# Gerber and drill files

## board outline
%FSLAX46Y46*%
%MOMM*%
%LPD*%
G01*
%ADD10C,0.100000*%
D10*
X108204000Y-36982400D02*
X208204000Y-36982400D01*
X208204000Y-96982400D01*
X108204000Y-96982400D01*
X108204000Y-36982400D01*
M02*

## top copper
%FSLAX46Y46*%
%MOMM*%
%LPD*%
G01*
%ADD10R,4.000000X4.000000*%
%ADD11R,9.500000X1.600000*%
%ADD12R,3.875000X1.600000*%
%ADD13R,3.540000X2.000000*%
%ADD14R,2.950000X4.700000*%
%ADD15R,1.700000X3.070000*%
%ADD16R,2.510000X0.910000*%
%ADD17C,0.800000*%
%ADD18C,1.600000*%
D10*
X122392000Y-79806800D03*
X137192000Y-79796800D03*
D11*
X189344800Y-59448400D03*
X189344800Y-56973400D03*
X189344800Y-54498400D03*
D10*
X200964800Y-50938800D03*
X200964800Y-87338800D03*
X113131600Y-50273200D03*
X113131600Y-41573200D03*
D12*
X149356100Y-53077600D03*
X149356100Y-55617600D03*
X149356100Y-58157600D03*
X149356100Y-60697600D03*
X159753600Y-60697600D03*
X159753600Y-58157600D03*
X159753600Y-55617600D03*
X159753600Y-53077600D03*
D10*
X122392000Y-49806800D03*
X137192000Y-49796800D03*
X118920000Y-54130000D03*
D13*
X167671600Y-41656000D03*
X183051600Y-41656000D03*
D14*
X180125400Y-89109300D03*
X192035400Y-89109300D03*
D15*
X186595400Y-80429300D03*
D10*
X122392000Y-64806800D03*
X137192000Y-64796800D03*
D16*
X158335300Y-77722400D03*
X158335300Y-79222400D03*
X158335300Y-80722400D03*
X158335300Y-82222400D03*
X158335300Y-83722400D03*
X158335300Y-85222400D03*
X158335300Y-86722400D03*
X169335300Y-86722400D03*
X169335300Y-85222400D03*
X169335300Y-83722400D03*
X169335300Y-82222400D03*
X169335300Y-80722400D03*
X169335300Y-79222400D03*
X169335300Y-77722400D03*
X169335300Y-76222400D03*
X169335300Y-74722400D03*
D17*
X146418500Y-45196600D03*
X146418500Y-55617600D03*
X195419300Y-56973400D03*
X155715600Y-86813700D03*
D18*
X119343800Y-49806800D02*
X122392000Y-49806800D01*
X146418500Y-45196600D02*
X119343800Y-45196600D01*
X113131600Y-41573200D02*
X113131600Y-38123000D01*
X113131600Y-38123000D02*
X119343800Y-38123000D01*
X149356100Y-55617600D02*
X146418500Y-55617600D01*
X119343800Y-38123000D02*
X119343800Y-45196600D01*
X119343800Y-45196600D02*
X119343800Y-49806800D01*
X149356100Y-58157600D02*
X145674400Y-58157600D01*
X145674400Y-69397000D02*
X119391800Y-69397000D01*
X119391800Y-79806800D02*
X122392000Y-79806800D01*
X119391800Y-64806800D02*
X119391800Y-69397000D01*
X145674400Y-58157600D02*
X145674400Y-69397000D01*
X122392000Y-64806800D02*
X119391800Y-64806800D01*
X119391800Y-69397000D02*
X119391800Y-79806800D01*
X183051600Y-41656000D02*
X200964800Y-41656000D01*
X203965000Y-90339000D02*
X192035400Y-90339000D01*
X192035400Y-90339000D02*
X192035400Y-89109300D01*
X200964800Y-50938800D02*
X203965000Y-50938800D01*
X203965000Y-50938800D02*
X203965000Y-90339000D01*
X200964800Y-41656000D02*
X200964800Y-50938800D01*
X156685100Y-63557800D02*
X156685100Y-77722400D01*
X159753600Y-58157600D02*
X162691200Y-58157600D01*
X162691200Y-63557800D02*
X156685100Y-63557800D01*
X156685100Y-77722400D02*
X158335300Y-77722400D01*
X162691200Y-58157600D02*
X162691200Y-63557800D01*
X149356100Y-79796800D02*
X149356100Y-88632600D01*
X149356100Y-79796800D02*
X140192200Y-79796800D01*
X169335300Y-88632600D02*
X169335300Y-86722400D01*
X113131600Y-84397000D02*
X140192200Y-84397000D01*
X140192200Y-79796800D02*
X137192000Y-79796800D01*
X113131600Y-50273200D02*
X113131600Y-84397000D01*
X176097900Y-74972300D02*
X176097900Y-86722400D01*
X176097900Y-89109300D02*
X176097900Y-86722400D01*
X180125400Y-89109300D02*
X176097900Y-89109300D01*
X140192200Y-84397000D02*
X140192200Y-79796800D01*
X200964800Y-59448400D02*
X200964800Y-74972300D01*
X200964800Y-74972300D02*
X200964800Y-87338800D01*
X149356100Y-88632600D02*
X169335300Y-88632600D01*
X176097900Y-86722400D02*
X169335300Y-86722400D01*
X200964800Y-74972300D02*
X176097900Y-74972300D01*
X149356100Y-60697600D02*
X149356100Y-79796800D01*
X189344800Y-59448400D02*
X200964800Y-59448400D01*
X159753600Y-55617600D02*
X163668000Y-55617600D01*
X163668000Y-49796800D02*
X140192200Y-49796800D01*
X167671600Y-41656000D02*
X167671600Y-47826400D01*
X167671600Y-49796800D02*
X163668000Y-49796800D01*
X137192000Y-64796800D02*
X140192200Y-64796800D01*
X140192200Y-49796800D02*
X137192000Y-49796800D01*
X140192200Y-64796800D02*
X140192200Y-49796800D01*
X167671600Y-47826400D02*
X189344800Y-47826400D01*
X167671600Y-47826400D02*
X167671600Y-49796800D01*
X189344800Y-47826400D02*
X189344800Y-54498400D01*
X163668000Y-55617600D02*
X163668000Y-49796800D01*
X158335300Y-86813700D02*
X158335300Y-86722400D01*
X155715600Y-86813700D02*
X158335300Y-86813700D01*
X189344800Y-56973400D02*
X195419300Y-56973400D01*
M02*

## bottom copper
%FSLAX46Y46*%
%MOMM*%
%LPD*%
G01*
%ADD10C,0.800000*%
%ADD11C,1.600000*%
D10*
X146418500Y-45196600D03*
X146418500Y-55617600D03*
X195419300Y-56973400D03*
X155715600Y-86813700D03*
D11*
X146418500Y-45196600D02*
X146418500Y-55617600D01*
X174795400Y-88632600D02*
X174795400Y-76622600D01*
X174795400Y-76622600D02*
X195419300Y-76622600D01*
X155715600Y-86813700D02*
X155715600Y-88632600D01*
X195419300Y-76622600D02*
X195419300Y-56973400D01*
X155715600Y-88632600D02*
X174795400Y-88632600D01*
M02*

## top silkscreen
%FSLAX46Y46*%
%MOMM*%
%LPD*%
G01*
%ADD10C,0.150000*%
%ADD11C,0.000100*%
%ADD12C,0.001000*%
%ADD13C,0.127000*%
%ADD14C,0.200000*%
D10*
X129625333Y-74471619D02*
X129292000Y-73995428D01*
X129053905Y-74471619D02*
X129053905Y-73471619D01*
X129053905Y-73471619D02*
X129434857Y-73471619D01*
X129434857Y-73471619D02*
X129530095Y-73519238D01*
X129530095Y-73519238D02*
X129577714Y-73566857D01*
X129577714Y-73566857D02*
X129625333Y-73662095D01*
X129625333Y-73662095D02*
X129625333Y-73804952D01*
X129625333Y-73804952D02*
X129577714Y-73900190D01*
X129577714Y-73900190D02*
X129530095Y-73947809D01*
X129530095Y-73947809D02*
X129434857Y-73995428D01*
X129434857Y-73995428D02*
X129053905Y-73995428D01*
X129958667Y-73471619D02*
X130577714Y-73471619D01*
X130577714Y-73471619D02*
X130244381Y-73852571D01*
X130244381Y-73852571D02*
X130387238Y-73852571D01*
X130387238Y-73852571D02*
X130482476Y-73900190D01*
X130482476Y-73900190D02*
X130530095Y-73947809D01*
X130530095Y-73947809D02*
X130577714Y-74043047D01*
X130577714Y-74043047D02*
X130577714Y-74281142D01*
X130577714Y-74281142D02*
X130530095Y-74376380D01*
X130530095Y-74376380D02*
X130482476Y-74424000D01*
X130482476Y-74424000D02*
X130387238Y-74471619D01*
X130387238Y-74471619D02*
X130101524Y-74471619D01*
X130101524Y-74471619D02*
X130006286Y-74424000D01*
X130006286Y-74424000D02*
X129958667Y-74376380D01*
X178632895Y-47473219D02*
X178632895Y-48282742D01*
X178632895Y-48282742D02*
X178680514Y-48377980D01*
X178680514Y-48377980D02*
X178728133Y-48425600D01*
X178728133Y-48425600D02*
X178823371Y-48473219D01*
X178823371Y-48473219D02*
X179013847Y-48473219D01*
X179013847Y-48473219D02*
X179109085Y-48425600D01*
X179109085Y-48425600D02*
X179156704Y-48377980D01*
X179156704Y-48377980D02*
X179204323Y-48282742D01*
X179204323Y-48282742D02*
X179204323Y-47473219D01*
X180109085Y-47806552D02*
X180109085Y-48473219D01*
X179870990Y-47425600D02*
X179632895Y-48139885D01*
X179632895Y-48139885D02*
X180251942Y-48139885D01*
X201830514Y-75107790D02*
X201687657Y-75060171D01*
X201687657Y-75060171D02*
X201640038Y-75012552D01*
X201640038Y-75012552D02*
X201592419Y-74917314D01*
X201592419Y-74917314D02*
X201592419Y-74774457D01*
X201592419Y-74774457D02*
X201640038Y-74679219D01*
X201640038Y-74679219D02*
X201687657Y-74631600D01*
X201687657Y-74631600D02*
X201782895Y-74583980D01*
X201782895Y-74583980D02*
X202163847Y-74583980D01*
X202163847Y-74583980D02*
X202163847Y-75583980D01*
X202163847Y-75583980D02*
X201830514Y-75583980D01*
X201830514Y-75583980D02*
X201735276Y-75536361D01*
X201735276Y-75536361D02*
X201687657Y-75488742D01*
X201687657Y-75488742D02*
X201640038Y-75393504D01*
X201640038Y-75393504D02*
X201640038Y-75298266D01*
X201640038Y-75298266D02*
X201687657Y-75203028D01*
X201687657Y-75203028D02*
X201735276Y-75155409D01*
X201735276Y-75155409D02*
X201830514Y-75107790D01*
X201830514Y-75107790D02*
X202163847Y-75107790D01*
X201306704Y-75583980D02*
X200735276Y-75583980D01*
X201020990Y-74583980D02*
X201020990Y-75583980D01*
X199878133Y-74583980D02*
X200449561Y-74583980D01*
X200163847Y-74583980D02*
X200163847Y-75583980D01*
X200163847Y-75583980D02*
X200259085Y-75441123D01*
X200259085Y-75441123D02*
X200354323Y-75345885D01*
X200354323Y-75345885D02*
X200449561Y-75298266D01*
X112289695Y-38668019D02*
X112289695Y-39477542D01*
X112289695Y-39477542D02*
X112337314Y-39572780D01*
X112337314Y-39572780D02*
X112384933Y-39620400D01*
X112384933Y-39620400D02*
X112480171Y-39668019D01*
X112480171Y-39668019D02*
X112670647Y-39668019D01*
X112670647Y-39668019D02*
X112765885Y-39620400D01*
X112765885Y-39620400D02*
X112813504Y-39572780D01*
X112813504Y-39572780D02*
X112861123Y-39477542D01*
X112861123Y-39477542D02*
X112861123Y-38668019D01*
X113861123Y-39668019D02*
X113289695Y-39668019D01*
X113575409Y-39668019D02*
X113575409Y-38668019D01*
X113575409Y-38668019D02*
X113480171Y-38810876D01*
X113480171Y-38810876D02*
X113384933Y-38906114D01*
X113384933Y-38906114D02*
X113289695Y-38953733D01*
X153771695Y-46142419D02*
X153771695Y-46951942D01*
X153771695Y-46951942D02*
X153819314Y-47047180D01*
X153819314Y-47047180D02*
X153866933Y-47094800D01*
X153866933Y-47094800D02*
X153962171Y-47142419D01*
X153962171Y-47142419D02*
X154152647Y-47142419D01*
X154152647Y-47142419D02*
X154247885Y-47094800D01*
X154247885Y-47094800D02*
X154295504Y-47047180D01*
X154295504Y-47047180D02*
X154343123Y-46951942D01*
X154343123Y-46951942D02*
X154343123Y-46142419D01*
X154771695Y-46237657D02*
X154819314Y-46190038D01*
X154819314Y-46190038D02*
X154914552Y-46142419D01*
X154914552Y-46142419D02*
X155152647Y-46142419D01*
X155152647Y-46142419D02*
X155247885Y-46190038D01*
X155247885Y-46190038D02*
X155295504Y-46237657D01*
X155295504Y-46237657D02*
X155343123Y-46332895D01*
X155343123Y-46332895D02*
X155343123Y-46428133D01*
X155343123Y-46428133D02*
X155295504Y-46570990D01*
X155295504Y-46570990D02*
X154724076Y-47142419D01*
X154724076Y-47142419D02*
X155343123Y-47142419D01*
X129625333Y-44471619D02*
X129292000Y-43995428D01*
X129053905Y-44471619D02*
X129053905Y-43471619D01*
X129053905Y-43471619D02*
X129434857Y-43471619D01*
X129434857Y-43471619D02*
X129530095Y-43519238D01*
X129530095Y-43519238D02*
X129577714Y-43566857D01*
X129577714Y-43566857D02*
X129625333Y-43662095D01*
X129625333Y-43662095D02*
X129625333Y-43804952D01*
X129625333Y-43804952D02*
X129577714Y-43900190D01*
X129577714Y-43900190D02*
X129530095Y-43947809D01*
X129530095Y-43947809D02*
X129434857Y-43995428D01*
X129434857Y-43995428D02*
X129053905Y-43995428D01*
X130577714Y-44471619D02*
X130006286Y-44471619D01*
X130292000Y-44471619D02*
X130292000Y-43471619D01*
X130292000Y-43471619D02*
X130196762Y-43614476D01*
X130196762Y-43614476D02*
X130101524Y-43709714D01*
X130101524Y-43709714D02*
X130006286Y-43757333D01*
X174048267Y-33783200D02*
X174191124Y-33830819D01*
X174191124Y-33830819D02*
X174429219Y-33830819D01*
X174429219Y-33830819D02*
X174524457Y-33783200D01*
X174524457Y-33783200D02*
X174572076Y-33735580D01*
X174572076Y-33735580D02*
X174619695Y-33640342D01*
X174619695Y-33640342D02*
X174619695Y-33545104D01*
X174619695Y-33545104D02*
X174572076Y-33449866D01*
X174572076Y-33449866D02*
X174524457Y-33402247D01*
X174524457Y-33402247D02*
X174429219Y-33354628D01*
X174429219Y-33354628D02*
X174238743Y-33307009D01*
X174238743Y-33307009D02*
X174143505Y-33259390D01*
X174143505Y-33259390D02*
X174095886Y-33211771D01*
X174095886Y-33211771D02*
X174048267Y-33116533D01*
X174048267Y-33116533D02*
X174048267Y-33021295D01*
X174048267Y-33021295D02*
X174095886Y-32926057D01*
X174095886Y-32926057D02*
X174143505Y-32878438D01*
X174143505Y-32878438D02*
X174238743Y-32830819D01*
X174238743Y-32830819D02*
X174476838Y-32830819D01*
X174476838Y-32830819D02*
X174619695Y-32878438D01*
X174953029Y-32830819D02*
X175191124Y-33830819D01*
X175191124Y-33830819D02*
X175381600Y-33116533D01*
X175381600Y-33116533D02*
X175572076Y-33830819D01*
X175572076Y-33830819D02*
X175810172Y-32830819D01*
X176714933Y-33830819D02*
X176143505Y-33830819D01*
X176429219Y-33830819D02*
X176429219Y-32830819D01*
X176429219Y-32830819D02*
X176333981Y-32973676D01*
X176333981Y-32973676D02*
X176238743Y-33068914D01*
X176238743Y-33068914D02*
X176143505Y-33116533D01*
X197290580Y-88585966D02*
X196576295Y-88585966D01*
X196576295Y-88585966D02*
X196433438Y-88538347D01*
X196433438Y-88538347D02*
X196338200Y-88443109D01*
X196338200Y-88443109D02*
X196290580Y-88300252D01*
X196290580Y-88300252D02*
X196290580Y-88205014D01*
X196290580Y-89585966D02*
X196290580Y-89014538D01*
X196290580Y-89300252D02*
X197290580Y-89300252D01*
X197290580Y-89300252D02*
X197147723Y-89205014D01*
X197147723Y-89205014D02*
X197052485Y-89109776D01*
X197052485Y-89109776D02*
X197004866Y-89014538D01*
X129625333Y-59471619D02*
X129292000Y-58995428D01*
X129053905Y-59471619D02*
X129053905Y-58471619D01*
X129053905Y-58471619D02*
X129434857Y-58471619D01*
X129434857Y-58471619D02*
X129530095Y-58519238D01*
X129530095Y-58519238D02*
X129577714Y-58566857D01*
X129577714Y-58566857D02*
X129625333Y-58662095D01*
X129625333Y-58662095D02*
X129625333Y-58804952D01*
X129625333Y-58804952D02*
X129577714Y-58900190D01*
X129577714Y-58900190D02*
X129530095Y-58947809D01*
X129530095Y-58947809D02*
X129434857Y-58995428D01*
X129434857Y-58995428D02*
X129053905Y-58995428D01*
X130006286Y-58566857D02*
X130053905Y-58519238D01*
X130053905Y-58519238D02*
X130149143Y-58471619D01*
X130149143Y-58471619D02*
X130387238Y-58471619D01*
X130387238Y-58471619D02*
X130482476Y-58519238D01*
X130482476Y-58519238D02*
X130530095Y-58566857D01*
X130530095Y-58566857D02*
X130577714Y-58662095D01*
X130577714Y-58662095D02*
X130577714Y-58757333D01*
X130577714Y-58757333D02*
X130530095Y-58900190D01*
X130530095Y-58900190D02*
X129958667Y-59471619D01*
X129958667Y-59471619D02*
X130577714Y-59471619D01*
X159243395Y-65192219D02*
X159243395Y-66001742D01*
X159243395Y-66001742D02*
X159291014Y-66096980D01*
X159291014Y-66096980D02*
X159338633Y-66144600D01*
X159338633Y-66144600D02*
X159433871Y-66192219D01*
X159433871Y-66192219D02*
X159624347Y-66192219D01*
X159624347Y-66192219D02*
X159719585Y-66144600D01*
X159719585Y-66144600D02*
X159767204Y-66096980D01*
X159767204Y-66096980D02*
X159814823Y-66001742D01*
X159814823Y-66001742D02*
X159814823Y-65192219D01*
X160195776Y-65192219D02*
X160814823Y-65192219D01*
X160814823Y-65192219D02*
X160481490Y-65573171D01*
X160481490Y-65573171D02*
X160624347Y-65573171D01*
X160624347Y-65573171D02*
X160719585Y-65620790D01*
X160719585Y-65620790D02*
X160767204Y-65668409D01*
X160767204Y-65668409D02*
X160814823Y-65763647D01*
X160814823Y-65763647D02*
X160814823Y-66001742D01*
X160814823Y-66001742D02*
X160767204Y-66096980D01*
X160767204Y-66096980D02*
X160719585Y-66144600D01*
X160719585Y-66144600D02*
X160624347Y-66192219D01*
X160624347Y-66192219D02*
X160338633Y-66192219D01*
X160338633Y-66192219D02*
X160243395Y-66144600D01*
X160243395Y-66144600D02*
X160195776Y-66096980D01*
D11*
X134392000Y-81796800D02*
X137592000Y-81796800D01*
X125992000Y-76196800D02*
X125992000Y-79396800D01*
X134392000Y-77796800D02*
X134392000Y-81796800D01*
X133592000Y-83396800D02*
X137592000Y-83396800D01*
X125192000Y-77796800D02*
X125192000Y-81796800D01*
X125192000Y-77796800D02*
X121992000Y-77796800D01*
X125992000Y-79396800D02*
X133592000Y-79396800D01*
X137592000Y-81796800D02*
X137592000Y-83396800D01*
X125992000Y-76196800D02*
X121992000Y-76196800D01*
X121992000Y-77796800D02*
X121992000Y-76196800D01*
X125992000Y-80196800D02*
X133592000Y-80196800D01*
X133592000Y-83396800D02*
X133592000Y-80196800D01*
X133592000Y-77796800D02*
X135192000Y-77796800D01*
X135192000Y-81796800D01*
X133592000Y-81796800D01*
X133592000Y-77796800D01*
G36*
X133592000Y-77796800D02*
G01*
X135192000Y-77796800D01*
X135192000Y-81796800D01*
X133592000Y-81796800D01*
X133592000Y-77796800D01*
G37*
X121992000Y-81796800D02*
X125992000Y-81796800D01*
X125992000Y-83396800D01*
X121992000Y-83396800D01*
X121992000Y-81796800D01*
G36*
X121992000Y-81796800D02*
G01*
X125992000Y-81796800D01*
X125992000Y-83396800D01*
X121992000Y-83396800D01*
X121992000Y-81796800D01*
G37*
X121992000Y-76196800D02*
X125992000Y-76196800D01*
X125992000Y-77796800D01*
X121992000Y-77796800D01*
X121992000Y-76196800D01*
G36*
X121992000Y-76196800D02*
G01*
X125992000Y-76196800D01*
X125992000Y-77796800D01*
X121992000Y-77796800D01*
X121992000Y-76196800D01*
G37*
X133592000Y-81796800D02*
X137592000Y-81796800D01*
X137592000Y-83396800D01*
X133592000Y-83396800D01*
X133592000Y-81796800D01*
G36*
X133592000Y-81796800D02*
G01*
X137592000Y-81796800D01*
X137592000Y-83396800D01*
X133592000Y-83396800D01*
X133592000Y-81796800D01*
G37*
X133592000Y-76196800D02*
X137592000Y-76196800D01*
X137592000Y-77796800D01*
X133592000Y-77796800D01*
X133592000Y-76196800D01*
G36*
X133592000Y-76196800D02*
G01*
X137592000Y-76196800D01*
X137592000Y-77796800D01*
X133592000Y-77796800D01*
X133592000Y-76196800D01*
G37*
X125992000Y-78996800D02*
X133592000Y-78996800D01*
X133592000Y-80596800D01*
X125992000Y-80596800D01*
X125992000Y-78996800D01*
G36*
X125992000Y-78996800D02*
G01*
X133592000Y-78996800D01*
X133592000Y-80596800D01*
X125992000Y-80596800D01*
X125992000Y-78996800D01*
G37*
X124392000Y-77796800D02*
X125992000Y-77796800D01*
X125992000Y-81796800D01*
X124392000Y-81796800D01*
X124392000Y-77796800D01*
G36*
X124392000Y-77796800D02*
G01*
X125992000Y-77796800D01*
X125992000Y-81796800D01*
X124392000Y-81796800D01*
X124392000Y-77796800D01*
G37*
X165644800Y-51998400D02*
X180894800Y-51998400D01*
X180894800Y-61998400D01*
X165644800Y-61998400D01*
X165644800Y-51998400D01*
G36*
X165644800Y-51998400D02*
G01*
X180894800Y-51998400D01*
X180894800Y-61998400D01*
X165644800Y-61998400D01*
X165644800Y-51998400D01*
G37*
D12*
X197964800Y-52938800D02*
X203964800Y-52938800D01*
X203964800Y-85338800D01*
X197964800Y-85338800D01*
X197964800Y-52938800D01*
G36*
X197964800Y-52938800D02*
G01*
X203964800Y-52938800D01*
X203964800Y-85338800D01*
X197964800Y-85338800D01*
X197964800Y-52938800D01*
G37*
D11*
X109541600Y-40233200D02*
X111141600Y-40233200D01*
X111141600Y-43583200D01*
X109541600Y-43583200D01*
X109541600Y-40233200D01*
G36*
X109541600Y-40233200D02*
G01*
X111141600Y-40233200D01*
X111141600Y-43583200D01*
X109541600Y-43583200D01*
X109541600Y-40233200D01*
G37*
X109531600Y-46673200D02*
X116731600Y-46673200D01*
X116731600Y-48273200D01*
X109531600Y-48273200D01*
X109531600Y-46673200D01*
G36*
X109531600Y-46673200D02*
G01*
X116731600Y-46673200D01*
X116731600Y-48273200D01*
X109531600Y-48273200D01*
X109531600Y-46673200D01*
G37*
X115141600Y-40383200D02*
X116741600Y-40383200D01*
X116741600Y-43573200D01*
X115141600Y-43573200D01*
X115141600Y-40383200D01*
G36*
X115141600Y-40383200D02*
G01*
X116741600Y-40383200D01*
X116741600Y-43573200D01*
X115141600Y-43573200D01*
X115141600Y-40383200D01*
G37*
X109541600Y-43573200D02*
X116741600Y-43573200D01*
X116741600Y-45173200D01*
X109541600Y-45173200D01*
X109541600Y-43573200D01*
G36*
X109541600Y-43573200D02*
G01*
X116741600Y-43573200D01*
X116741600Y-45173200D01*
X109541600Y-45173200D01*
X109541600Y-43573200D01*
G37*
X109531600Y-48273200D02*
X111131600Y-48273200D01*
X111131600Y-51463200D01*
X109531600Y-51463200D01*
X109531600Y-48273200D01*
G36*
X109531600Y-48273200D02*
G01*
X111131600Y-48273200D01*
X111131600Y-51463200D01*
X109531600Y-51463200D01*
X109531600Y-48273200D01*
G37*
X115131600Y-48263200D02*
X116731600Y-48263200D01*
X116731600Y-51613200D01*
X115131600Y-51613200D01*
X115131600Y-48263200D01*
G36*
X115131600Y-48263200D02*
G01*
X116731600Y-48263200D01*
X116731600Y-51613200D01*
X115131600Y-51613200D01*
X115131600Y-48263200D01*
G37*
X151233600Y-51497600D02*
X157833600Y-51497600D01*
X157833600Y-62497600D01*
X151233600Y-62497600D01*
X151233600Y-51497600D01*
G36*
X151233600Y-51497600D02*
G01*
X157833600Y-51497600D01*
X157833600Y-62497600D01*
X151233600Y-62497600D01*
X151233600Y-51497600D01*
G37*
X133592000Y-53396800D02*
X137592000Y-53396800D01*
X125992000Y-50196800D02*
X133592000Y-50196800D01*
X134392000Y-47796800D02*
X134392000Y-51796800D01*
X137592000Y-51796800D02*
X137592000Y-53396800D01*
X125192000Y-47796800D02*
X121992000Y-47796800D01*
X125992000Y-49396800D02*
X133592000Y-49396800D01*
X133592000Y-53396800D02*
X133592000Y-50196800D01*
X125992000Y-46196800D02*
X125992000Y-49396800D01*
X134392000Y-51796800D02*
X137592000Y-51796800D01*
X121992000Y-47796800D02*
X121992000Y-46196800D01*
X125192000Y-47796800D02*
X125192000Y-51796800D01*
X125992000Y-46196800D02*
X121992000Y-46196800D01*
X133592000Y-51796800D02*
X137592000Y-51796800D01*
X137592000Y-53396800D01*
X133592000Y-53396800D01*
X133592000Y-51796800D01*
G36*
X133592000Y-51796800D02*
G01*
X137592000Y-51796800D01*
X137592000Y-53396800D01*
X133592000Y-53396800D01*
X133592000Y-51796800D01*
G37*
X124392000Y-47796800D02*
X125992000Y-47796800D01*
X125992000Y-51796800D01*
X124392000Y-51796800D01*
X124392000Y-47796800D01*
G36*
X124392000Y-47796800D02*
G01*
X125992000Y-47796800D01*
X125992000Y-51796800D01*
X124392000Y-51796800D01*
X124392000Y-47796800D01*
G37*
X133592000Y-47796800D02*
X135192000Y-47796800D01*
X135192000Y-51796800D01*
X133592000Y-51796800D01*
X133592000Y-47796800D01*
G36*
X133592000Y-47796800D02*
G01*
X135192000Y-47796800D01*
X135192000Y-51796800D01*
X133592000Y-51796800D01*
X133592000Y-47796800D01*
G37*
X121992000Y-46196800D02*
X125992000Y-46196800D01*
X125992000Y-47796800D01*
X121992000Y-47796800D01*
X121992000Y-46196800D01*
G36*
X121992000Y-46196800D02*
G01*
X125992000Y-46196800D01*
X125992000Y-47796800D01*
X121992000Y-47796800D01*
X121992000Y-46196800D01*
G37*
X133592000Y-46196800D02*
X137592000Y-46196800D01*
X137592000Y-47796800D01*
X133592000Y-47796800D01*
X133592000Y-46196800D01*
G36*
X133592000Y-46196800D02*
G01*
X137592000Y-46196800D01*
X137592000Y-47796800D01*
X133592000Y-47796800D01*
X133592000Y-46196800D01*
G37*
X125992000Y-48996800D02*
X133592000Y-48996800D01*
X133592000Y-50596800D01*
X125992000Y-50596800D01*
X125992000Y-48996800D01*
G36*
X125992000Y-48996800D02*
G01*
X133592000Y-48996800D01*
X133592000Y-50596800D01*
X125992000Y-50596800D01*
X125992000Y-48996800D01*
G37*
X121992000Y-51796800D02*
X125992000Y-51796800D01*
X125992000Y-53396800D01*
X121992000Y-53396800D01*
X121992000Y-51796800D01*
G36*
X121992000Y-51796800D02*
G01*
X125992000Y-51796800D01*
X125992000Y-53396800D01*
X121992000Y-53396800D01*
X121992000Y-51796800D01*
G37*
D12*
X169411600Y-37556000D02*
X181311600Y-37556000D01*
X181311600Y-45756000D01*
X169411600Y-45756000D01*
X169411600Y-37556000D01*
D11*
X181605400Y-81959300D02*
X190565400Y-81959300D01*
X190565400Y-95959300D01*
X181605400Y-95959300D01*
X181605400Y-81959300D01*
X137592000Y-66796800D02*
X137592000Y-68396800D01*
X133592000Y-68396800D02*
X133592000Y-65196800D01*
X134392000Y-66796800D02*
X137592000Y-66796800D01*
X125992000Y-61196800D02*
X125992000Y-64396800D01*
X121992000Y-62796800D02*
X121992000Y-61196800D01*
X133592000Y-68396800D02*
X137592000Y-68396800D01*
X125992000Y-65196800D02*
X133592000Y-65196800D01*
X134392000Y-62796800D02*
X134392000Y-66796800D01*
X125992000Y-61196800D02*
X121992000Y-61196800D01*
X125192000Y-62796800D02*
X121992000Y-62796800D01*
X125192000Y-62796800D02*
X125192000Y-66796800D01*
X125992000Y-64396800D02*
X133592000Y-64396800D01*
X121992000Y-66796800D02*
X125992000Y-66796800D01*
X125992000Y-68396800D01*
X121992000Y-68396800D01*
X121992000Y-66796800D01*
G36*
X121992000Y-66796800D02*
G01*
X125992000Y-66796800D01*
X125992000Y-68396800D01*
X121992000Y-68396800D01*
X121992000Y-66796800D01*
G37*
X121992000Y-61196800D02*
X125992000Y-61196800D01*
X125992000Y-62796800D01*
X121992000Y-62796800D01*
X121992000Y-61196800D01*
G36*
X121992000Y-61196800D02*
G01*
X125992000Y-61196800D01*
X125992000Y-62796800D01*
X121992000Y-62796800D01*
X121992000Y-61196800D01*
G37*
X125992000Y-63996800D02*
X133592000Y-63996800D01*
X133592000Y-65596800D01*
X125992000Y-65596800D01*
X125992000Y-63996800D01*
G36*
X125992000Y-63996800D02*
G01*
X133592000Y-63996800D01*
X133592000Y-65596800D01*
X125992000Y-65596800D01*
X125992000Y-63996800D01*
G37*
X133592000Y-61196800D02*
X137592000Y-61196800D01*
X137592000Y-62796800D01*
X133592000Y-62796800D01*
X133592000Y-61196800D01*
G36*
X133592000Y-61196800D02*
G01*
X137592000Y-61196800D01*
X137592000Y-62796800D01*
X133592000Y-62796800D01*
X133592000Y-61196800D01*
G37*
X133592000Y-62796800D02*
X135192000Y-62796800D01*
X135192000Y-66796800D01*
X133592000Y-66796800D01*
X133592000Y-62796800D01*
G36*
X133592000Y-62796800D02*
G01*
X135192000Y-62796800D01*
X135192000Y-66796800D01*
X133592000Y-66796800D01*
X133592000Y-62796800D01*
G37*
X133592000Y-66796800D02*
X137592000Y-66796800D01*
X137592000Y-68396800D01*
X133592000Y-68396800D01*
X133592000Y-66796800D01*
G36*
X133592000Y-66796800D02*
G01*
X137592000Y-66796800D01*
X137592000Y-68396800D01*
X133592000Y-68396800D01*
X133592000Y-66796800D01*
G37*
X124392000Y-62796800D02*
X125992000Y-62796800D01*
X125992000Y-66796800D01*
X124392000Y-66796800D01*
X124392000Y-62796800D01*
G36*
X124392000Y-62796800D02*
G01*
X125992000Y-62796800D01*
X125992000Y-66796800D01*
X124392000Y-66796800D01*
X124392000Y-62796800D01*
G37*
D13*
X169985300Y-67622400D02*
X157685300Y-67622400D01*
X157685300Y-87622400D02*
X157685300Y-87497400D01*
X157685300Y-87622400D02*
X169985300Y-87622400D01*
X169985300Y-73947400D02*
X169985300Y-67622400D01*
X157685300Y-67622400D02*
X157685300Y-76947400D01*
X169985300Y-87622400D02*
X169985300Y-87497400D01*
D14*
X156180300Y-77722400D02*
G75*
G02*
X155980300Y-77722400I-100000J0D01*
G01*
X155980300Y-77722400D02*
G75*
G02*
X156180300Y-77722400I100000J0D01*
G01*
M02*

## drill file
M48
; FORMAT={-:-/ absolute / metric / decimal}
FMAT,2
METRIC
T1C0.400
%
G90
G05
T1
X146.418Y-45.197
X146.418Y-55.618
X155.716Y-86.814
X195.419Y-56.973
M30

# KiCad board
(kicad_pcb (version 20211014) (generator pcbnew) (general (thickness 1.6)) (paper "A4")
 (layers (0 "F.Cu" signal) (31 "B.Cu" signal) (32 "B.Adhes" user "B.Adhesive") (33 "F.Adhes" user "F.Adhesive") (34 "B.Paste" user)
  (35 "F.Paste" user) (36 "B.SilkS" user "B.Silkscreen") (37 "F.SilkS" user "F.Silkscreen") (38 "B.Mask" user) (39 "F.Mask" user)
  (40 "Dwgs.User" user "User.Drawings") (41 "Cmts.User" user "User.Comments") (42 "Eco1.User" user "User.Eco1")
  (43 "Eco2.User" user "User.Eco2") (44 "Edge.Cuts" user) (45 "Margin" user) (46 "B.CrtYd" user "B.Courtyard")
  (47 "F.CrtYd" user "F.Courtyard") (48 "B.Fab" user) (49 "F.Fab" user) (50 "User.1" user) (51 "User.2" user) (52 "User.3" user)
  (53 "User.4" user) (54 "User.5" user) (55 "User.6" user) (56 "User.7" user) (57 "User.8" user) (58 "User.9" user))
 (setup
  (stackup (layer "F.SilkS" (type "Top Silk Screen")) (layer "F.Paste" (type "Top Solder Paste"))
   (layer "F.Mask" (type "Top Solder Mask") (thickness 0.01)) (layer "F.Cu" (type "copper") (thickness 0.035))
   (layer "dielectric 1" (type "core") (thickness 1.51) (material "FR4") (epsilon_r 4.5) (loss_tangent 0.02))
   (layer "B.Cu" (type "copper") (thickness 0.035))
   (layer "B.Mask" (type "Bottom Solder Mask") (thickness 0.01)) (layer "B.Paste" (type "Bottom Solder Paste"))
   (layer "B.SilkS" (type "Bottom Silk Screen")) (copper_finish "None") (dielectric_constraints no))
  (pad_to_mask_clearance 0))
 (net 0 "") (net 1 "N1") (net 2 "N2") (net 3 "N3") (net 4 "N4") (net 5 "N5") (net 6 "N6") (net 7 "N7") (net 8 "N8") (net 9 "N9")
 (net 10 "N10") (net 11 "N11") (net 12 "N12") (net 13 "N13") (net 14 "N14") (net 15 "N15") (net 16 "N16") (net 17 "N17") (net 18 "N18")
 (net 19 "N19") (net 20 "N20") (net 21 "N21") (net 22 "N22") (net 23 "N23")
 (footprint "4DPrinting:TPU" (layer "F.Cu") (at 129.792 79.7968)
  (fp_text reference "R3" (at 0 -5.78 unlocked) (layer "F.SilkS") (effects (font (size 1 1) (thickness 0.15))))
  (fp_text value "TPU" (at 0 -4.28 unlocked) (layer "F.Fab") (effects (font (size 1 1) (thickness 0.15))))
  (fp_line (start 4.6 2) (end 7.8 2) (layer "F.SilkS") (width 0.0001))
  (fp_line (start -3.8 -3.6) (end -3.8 -0.4) (layer "F.SilkS") (width 0.0001))
  (fp_line (start 4.6 -2) (end 4.6 2) (layer "F.SilkS") (width 0.0001))
  (fp_line (start 3.8 3.6) (end 7.8 3.6) (layer "F.SilkS") (width 0.0001))
  (fp_line (start -4.6 -2) (end -4.6 2) (layer "F.SilkS") (width 0.0001))
  (fp_line (start -4.6 -2) (end -7.8 -2) (layer "F.SilkS") (width 0.0001))
  (fp_line (start -3.8 -0.4) (end 3.8 -0.4) (layer "F.SilkS") (width 0.0001))
  (fp_line (start 7.8 2) (end 7.8 3.6) (layer "F.SilkS") (width 0.0001))
  (fp_line (start -3.8 -3.6) (end -7.8 -3.6) (layer "F.SilkS") (width 0.0001))
  (fp_line (start -7.8 -2) (end -7.8 -3.6) (layer "F.SilkS") (width 0.0001))
  (fp_line (start -3.8 0.4) (end 3.8 0.4) (layer "F.SilkS") (width 0.0001))
  (fp_line (start 3.8 3.6) (end 3.8 0.4) (layer "F.SilkS") (width 0.0001))
  (fp_rect (start 3.8 -2) (end 5.4 2) (layer "F.SilkS") (width 0.0001) (fill solid))
  (fp_rect (start -7.8 2) (end -3.8 3.6) (layer "F.SilkS") (width 0.0001) (fill solid))
  (fp_rect (start -7.8 -3.6) (end -3.8 -2) (layer "F.SilkS") (width 0.0001) (fill solid))
  (fp_rect (start 3.8 2) (end 7.8 3.6) (layer "F.SilkS") (width 0.0001) (fill solid))
  (fp_rect (start 3.8 -3.6) (end 7.8 -2) (layer "F.SilkS") (width 0.0001) (fill solid))
  (fp_rect (start -3.8 -0.8) (end 3.8 0.8) (layer "F.SilkS") (width 0.0001) (fill solid))
  (fp_rect (start -5.4 -2) (end -3.8 2) (layer "F.SilkS") (width 0.0001) (fill solid))
  (pad "1" smd rect (at -7.4 0.01) (size 4 4) (layers "F.Cu" "F.Paste" "F.Mask") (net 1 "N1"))
  (pad "2" smd rect (at 7.4 0) (size 4 4) (layers "F.Cu" "F.Paste" "F.Mask") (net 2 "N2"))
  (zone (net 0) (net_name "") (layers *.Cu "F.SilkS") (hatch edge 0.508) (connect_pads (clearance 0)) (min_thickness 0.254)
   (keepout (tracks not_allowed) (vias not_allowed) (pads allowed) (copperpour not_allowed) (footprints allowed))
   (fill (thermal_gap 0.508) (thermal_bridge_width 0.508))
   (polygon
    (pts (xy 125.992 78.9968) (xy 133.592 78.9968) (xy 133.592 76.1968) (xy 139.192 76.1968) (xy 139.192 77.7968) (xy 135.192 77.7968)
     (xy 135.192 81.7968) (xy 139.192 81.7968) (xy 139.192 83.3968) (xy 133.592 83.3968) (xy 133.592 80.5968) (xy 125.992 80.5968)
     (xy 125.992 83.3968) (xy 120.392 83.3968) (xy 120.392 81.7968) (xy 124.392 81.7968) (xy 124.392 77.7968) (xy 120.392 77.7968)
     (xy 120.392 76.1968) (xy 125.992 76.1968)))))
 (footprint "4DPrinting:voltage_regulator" (layer "F.Cu") (at 179.3748 57.0484)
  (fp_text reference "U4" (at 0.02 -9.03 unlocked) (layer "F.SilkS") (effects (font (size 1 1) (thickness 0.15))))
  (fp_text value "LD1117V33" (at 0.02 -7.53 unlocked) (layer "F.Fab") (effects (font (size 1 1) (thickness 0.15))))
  (fp_rect (start -13.73 -5.05) (end 1.52 4.95) (layer "F.SilkS") (width 0.0001) (fill solid))
  (pad "1" smd rect (at 9.97 2.4) (size 9.5 1.6) (layers "F.Cu" "F.Paste" "F.Mask") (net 2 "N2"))
  (pad "2" smd rect (at 9.97 -0.075) (size 9.5 1.6) (layers "F.Cu" "F.Paste" "F.Mask") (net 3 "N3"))
  (pad "3" smd rect (at 9.97 -2.55) (size 9.5 1.6) (layers "F.Cu" "F.Paste" "F.Mask") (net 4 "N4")))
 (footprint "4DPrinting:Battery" (layer "F.Cu") (at 200.9648 69.1388 180)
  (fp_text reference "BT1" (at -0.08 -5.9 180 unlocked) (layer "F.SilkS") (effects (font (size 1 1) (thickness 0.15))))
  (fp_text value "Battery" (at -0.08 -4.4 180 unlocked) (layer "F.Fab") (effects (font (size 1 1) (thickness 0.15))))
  (fp_rect (start -3 -16.2) (end 3 16.2) (layer "F.SilkS") (width 0.001) (fill solid))
  (pad "1" smd rect (at 0 18.2 180) (size 4 4) (layers "F.Cu" "F.Paste" "F.Mask") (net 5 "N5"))
  (pad "2" smd rect (at 0 -18.2 180) (size 4 4) (layers "F.Cu" "F.Paste" "F.Mask") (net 2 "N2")))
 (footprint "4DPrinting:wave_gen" (layer "F.Cu") (at 113.1316 45.9232)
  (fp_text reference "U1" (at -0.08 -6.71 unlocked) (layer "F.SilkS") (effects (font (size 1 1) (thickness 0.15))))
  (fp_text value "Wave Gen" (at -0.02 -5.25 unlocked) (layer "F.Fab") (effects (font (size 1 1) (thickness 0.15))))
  (fp_rect (start -3.59 -2.34) (end -1.99 -5.69) (layer "F.SilkS") (width 0.0001) (fill solid))
  (fp_rect (start -3.6 0.75) (end 3.6 2.35) (layer "F.SilkS") (width 0.0001) (fill solid))
  (fp_rect (start 2.01 -2.35) (end 3.61 -5.54) (layer "F.SilkS") (width 0.0001) (fill solid))
  (fp_rect (start 3.61 -0.75) (end -3.59 -2.35) (layer "F.SilkS") (width 0.0001) (fill solid))
  (fp_rect (start -2 2.35) (end -3.6 5.54) (layer "F.SilkS") (width 0.0001) (fill solid))
  (fp_rect (start 3.6 2.34) (end 2 5.69) (layer "F.SilkS") (width 0.0001) (fill solid))
  (pad "1" smd rect (at 0 4.35) (size 4 4) (layers "F.Cu" "F.Paste" "F.Mask") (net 2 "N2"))
  (pad "2" smd rect (at 0 -4.35 180) (size 4 4) (layers "F.Cu" "F.Paste" "F.Mask") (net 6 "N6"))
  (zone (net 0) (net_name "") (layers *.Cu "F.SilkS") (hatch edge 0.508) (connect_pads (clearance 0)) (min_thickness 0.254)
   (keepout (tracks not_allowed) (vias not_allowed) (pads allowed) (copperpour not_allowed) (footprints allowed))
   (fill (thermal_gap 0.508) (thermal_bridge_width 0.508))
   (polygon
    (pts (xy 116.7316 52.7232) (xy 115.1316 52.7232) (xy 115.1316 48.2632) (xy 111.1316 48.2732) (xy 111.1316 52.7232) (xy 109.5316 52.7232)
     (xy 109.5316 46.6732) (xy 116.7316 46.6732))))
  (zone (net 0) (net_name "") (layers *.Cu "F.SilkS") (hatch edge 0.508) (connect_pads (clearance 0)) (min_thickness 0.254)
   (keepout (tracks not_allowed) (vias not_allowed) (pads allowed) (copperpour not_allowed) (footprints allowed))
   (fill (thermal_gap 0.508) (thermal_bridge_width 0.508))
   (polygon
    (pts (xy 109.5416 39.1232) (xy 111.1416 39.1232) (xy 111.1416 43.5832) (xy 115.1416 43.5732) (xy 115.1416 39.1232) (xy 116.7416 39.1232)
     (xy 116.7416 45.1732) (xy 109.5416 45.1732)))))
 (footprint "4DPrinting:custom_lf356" (layer "F.Cu") (at 154.5336 56.9976)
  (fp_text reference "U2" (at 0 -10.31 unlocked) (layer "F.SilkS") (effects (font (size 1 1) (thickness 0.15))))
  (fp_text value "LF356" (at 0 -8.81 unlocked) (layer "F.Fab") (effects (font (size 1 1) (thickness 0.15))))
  (fp_rect (start -3.3 -5.5) (end 3.3 5.5) (layer "F.SilkS") (width 0.0001) (fill solid))
  (pad "1" smd rect (at -5.1775 -3.92) (size 3.875 1.6) (layers "F.Cu" "F.Paste" "F.Mask") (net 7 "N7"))
  (pad "2" smd rect (at -5.1775 -1.38) (size 3.875 1.6) (layers "F.Cu" "F.Paste" "F.Mask") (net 6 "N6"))
  (pad "3" smd rect (at -5.1775 1.16) (size 3.875 1.6) (layers "F.Cu" "F.Paste" "F.Mask") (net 1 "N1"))
  (pad "4" smd rect (at -5.1775 3.7) (size 3.875 1.6) (layers "F.Cu" "F.Paste" "F.Mask") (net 2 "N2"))
  (pad "5" smd rect (at 5.22 3.7) (size 3.875 1.6) (layers "F.Cu" "F.Paste" "F.Mask") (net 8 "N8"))
  (pad "6" smd rect (at 5.22 1.16) (size 3.875 1.6) (layers "F.Cu" "F.Paste" "F.Mask") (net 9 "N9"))
  (pad "7" smd rect (at 5.22 -1.38) (size 3.875 1.6) (layers "F.Cu" "F.Paste" "F.Mask") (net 4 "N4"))
  (pad "8" smd rect (at 5.22 -3.92) (size 3.875 1.6) (layers "F.Cu" "F.Paste" "F.Mask") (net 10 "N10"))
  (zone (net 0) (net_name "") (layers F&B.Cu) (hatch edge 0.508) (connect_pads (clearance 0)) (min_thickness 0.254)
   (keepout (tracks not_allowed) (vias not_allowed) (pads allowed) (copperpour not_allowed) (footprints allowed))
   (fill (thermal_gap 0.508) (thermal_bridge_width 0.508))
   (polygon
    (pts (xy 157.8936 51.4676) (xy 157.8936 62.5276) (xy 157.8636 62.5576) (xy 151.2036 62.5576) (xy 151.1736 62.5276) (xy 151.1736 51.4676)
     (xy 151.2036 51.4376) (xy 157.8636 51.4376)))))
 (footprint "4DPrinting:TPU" (layer "F.Cu") (at 129.792 49.7968)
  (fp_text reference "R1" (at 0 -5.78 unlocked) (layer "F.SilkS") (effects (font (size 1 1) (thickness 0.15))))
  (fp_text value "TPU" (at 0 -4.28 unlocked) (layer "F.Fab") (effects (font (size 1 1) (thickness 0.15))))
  (fp_line (start 3.8 3.6) (end 7.8 3.6) (layer "F.SilkS") (width 0.0001))
  (fp_line (start -3.8 0.4) (end 3.8 0.4) (layer "F.SilkS") (width 0.0001))
  (fp_line (start 4.6 -2) (end 4.6 2) (layer "F.SilkS") (width 0.0001))
  (fp_line (start 7.8 2) (end 7.8 3.6) (layer "F.SilkS") (width 0.0001))
  (fp_line (start -4.6 -2) (end -7.8 -2) (layer "F.SilkS") (width 0.0001))
  (fp_line (start -3.8 -0.4) (end 3.8 -0.4) (layer "F.SilkS") (width 0.0001))
  (fp_line (start 3.8 3.6) (end 3.8 0.4) (layer "F.SilkS") (width 0.0001))
  (fp_line (start -3.8 -3.6) (end -3.8 -0.4) (layer "F.SilkS") (width 0.0001))
  (fp_line (start 4.6 2) (end 7.8 2) (layer "F.SilkS") (width 0.0001))
  (fp_line (start -7.8 -2) (end -7.8 -3.6) (layer "F.SilkS") (width 0.0001))
  (fp_line (start -4.6 -2) (end -4.6 2) (layer "F.SilkS") (width 0.0001))
  (fp_line (start -3.8 -3.6) (end -7.8 -3.6) (layer "F.SilkS") (width 0.0001))
  (fp_rect (start 3.8 2) (end 7.8 3.6) (layer "F.SilkS") (width 0.0001) (fill solid))
  (fp_rect (start -5.4 -2) (end -3.8 2) (layer "F.SilkS") (width 0.0001) (fill solid))
  (fp_rect (start 3.8 -2) (end 5.4 2) (layer "F.SilkS") (width 0.0001) (fill solid))
  (fp_rect (start -7.8 -3.6) (end -3.8 -2) (layer "F.SilkS") (width 0.0001) (fill solid))
  (fp_rect (start 3.8 -3.6) (end 7.8 -2) (layer "F.SilkS") (width 0.0001) (fill solid))
  (fp_rect (start -3.8 -0.8) (end 3.8 0.8) (layer "F.SilkS") (width 0.0001) (fill solid))
  (fp_rect (start -7.8 2) (end -3.8 3.6) (layer "F.SilkS") (width 0.0001) (fill solid))
  (pad "1" smd rect (at -7.4 0.01) (size 4 4) (layers "F.Cu" "F.Paste" "F.Mask") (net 6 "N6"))
  (pad "2" smd rect (at 7.4 0) (size 4 4) (layers "F.Cu" "F.Paste" "F.Mask") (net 4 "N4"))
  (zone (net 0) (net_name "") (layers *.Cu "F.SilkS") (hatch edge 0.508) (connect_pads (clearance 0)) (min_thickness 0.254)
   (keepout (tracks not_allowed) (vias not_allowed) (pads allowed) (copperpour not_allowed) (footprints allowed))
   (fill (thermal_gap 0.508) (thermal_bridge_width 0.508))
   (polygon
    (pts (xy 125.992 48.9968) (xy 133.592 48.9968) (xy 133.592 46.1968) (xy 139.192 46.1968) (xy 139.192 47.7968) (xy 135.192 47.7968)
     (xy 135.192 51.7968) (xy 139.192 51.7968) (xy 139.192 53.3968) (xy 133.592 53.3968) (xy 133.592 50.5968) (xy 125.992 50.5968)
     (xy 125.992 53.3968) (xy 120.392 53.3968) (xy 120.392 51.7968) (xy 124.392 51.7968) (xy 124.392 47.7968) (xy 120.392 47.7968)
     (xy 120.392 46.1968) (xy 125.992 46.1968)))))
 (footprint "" (layer "F.Cu") (at 118.92 54.13)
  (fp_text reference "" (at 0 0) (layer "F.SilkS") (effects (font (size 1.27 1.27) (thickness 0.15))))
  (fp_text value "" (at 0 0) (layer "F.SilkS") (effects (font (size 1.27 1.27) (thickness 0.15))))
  (pad "1" smd rect (at 0 0) (size 4 4) (layers "F.Cu" "F.Paste" "F.Mask") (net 2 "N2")))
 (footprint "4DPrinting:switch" (layer "F.Cu") (at 175.3616 41.656)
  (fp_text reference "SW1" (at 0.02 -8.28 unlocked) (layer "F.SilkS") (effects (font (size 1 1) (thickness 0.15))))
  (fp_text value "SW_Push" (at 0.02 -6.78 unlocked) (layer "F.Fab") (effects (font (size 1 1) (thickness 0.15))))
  (fp_rect (start -5.95 4.1) (end 5.95 -4.1) (layer "F.SilkS") (width 0.001) (fill none))
  (pad "1" smd rect (at -7.69 0) (size 3.54 2) (layers "F.Cu" "F.Paste" "F.Mask") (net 4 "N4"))
  (pad "2" smd rect (at 7.69 0) (size 3.54 2) (layers "F.Cu" "F.Paste" "F.Mask") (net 5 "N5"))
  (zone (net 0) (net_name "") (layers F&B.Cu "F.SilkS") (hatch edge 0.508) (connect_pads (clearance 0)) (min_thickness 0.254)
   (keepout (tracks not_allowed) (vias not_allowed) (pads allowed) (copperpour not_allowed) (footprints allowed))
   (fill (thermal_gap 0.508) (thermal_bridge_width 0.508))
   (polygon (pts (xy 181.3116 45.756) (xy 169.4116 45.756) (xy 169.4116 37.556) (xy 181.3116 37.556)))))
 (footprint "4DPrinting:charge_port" (layer "F.Cu") (at 186.0854 88.9593 -90)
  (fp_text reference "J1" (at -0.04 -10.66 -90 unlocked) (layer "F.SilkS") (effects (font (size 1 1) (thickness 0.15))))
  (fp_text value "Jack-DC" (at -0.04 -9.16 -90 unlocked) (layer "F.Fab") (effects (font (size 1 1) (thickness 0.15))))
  (fp_rect (start -7 -4.48) (end 7 4.48) (layer "F.SilkS") (width 0.0001) (fill none))
  (pad "1" smd rect (at 0.15 5.96 90) (size 4.7 2.95) (layers "F.Cu" "F.Paste" "F.Mask") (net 5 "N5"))
  (pad "2" smd rect (at 0.15 -5.95 90) (size 4.7 2.95) (layers "F.Cu" "F.Paste" "F.Mask") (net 2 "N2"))
  (pad "3" smd rect (at -8.53 -0.51 90) (size 3.07 1.7) (layers "F.Cu" "F.Paste" "F.Mask")))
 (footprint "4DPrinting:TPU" (layer "F.Cu") (at 129.792 64.7968)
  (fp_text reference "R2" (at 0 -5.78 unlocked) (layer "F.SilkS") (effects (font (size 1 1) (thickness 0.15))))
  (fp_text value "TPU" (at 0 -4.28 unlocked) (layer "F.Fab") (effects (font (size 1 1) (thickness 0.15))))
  (fp_line (start 7.8 2) (end 7.8 3.6) (layer "F.SilkS") (width 0.0001))
  (fp_line (start 3.8 3.6) (end 3.8 0.4) (layer "F.SilkS") (width 0.0001))
  (fp_line (start 4.6 2) (end 7.8 2) (layer "F.SilkS") (width 0.0001))
  (fp_line (start -3.8 -3.6) (end -3.8 -0.4) (layer "F.SilkS") (width 0.0001))
  (fp_line (start -7.8 -2) (end -7.8 -3.6) (layer "F.SilkS") (width 0.0001))
  (fp_line (start 3.8 3.6) (end 7.8 3.6) (layer "F.SilkS") (width 0.0001))
  (fp_line (start -3.8 0.4) (end 3.8 0.4) (layer "F.SilkS") (width 0.0001))
  (fp_line (start 4.6 -2) (end 4.6 2) (layer "F.SilkS") (width 0.0001))
  (fp_line (start -3.8 -3.6) (end -7.8 -3.6) (layer "F.SilkS") (width 0.0001))
  (fp_line (start -4.6 -2) (end -7.8 -2) (layer "F.SilkS") (width 0.0001))
  (fp_line (start -4.6 -2) (end -4.6 2) (layer "F.SilkS") (width 0.0001))
  (fp_line (start -3.8 -0.4) (end 3.8 -0.4) (layer "F.SilkS") (width 0.0001))
  (fp_rect (start -7.8 2) (end -3.8 3.6) (layer "F.SilkS") (width 0.0001) (fill solid))
  (fp_rect (start -7.8 -3.6) (end -3.8 -2) (layer "F.SilkS") (width 0.0001) (fill solid))
  (fp_rect (start -3.8 -0.8) (end 3.8 0.8) (layer "F.SilkS") (width 0.0001) (fill solid))
  (fp_rect (start 3.8 -3.6) (end 7.8 -2) (layer "F.SilkS") (width 0.0001) (fill solid))
  (fp_rect (start 3.8 -2) (end 5.4 2) (layer "F.SilkS") (width 0.0001) (fill solid))
  (fp_rect (start 3.8 2) (end 7.8 3.6) (layer "F.SilkS") (width 0.0001) (fill solid))
  (fp_rect (start -5.4 -2) (end -3.8 2) (layer "F.SilkS") (width 0.0001) (fill solid))
  (pad "1" smd rect (at -7.4 0.01) (size 4 4) (layers "F.Cu" "F.Paste" "F.Mask") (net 1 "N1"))
  (pad "2" smd rect (at 7.4 0) (size 4 4) (layers "F.Cu" "F.Paste" "F.Mask") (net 4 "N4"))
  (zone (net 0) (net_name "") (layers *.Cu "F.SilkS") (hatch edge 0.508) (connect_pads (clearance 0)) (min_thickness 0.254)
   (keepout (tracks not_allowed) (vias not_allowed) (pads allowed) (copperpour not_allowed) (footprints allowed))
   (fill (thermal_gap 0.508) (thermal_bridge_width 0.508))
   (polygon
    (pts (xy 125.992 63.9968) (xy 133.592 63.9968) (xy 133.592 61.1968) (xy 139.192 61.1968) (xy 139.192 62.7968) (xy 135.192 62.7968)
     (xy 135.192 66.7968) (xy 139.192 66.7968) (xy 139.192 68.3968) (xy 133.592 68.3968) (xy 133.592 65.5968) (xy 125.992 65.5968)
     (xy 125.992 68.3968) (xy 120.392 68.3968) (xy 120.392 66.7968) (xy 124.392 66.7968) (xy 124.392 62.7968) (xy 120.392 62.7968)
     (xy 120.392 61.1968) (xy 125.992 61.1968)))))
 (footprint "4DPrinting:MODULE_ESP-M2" (layer "F.Cu") (at 163.8353 77.6224)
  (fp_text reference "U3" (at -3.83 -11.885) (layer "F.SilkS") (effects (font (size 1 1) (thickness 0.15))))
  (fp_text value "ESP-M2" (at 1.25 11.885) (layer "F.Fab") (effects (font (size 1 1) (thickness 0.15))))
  (fp_line (start 6.15 -10) (end -6.15 -10) (layer "F.SilkS") (width 0.127))
  (fp_line (start -6.15 10) (end -6.15 9.875) (layer "F.SilkS") (width 0.127))
  (fp_line (start -6.15 10) (end 6.15 10) (layer "F.SilkS") (width 0.127))
  (fp_line (start 6.15 -3.675) (end 6.15 -10) (layer "F.SilkS") (width 0.127))
  (fp_line (start -6.15 -10) (end -6.15 -0.675) (layer "F.SilkS") (width 0.127))
  (fp_line (start 6.15 10) (end 6.15 9.875) (layer "F.SilkS") (width 0.127))
  (fp_circle (center -7.755 0.1) (end -7.655 0.1) (layer "F.SilkS") (width 0.2) (fill none))
  (pad "1" smd rect (at -5.5 0.1) (size 2.51 0.91) (layers "F.Cu" "F.Paste" "F.Mask") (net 9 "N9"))
  (pad "2" smd rect (at -5.5 1.6) (size 2.51 0.91) (layers "F.Cu" "F.Paste" "F.Mask") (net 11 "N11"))
  (pad "3" smd rect (at -5.5 3.1) (size 2.51 0.91) (layers "F.Cu" "F.Paste" "F.Mask") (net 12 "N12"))
  (pad "4" smd rect (at -5.5 4.6) (size 2.51 0.91) (layers "F.Cu" "F.Paste" "F.Mask") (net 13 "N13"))
  (pad "5" smd rect (at -5.5 6.1) (size 2.51 0.91) (layers "F.Cu" "F.Paste" "F.Mask") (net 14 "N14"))
  (pad "6" smd rect (at -5.5 7.6) (size 2.51 0.91) (layers "F.Cu" "F.Paste" "F.Mask") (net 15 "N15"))
  (pad "7" smd rect (at -5.5 9.1) (size 2.51 0.91) (layers "F.Cu" "F.Paste" "F.Mask") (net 3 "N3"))
  (pad "8" smd rect (at 5.5 9.1) (size 2.51 0.91) (layers "F.Cu" "F.Paste" "F.Mask") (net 2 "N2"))
  (pad "9" smd rect (at 5.5 7.6) (size 2.51 0.91) (layers "F.Cu" "F.Paste" "F.Mask") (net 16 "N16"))
  (pad "10" smd rect (at 5.5 6.1) (size 2.51 0.91) (layers "F.Cu" "F.Paste" "F.Mask") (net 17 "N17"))
  (pad "11" smd rect (at 5.5 4.6) (size 2.51 0.91) (layers "F.Cu" "F.Paste" "F.Mask") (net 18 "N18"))
  (pad "12" smd rect (at 5.5 3.1) (size 2.51 0.91) (layers "F.Cu" "F.Paste" "F.Mask") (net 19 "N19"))
  (pad "13" smd rect (at 5.5 1.6) (size 2.51 0.91) (layers "F.Cu" "F.Paste" "F.Mask") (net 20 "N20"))
  (pad "14" smd rect (at 5.5 0.1) (size 2.51 0.91) (layers "F.Cu" "F.Paste" "F.Mask") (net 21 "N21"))
  (pad "15" smd rect (at 5.5 -1.4) (size 2.51 0.91) (layers "F.Cu" "F.Paste" "F.Mask") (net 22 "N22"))
  (pad "16" smd rect (at 5.5 -2.9) (size 2.51 0.91) (layers "F.Cu" "F.Paste" "F.Mask") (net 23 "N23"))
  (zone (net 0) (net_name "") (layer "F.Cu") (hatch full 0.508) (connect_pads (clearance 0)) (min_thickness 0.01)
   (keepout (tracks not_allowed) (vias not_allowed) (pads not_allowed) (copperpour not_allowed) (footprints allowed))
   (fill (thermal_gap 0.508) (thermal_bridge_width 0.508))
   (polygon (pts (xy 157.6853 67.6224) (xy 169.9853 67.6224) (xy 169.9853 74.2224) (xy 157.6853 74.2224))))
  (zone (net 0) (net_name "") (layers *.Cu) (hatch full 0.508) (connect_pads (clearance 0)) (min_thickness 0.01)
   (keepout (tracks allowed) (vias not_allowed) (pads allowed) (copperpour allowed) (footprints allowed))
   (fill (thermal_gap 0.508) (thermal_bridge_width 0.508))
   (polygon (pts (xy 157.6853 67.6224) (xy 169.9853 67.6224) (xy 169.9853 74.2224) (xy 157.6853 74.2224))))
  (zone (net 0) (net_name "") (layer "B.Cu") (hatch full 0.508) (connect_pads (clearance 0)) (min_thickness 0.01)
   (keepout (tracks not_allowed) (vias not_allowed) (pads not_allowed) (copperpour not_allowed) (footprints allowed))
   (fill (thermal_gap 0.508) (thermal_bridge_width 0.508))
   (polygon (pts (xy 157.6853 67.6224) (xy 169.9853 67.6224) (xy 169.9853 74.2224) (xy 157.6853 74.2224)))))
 (gr_rect (start 108.204 36.9824) (end 208.204 96.9824) (layer "Edge.Cuts") (width 0.1) (fill none))
 (segment (start 119.3438 49.8068) (end 122.392 49.8068) (width 1.6) (layer "F.Cu") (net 6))
 (segment (start 146.4185 45.1966) (end 119.3438 45.1966) (width 1.6) (layer "F.Cu") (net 6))
 (segment (start 113.1316 41.5732) (end 113.1316 38.123) (width 1.6) (layer "F.Cu") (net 6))
 (segment (start 113.1316 38.123) (end 119.3438 38.123) (width 1.6) (layer "F.Cu") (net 6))
 (segment (start 149.3561 55.6176) (end 146.4185 55.6176) (width 1.6) (layer "F.Cu") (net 6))
 (segment (start 119.3438 38.123) (end 119.3438 45.1966) (width 1.6) (layer "F.Cu") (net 6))
 (segment (start 119.3438 45.1966) (end 119.3438 49.8068) (width 1.6) (layer "F.Cu") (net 6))
 (via (at 146.4185 45.1966) (size 0.8) (drill 0.4) (layers "F.Cu" "B.Cu") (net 6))
 (via (at 146.4185 55.6176) (size 0.8) (drill 0.4) (layers "F.Cu" "B.Cu") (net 6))
 (segment (start 146.4185 45.1966) (end 146.4185 55.6176) (width 1.6) (layer "B.Cu") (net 6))
 (segment (start 149.3561 58.1576) (end 145.6744 58.1576) (width 1.6) (layer "F.Cu") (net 1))
 (segment (start 145.6744 69.397) (end 119.3918 69.397) (width 1.6) (layer "F.Cu") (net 1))
 (segment (start 119.3918 79.8068) (end 122.392 79.8068) (width 1.6) (layer "F.Cu") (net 1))
 (segment (start 119.3918 64.8068) (end 119.3918 69.397) (width 1.6) (layer "F.Cu") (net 1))
 (segment (start 145.6744 58.1576) (end 145.6744 69.397) (width 1.6) (layer "F.Cu") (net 1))
 (segment (start 122.392 64.8068) (end 119.3918 64.8068) (width 1.6) (layer "F.Cu") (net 1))
 (segment (start 119.3918 69.397) (end 119.3918 79.8068) (width 1.6) (layer "F.Cu") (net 1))
 (segment (start 183.0516 41.656) (end 200.9648 41.656) (width 1.6) (layer "F.Cu") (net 5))
 (segment (start 203.965 90.339) (end 192.0354 90.339) (width 1.6) (layer "F.Cu") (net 5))
 (segment (start 192.0354 90.339) (end 192.0354 89.1093) (width 1.6) (layer "F.Cu") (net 5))
 (segment (start 200.9648 50.9388) (end 203.965 50.9388) (width 1.6) (layer "F.Cu") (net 5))
 (segment (start 203.965 50.9388) (end 203.965 90.339) (width 1.6) (layer "F.Cu") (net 5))
 (segment (start 200.9648 41.656) (end 200.9648 50.9388) (width 1.6) (layer "F.Cu") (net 5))
 (segment (start 156.6851 63.5578) (end 156.6851 77.7224) (width 1.6) (layer "F.Cu") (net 9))
 (segment (start 159.7536 58.1576) (end 162.6912 58.1576) (width 1.6) (layer "F.Cu") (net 9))
 (segment (start 162.6912 63.5578) (end 156.6851 63.5578) (width 1.6) (layer "F.Cu") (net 9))
 (segment (start 156.6851 77.7224) (end 158.3353 77.7224) (width 1.6) (layer "F.Cu") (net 9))
 (segment (start 162.6912 58.1576) (end 162.6912 63.5578) (width 1.6) (layer "F.Cu") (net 9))
 (segment (start 149.3561 79.7968) (end 149.3561 88.6326) (width 1.6) (layer "F.Cu") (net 2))
 (segment (start 149.3561 79.7968) (end 140.1922 79.7968) (width 1.6) (layer "F.Cu") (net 2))
 (segment (start 169.3353 88.6326) (end 169.3353 86.7224) (width 1.6) (layer "F.Cu") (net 2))
 (segment (start 113.1316 84.397) (end 140.1922 84.397) (width 1.6) (layer "F.Cu") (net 2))
 (segment (start 140.1922 79.7968) (end 137.192 79.7968) (width 1.6) (layer "F.Cu") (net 2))
 (segment (start 113.1316 50.2732) (end 113.1316 84.397) (width 1.6) (layer "F.Cu") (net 2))
 (segment (start 176.0979 74.9723) (end 176.0979 86.7224) (width 1.6) (layer "F.Cu") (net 2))
 (segment (start 176.0979 89.1093) (end 176.0979 86.7224) (width 1.6) (layer "F.Cu") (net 2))
 (segment (start 180.1254 89.1093) (end 176.0979 89.1093) (width 1.6) (layer "F.Cu") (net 2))
 (segment (start 140.1922 84.397) (end 140.1922 79.7968) (width 1.6) (layer "F.Cu") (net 2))
 (segment (start 200.9648 59.4484) (end 200.9648 74.9723) (width 1.6) (layer "F.Cu") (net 2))
 (segment (start 200.9648 74.9723) (end 200.9648 87.3388) (width 1.6) (layer "F.Cu") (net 2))
 (segment (start 149.3561 88.6326) (end 169.3353 88.6326) (width 1.6) (layer "F.Cu") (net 2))
 (segment (start 176.0979 86.7224) (end 169.3353 86.7224) (width 1.6) (layer "F.Cu") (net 2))
 (segment (start 200.9648 74.9723) (end 176.0979 74.9723) (width 1.6) (layer "F.Cu") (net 2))
 (segment (start 149.3561 60.6976) (end 149.3561 79.7968) (width 1.6) (layer "F.Cu") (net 2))
 (segment (start 189.3448 59.4484) (end 200.9648 59.4484) (width 1.6) (layer "F.Cu") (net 2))
 (segment (start 159.7536 55.6176) (end 163.668 55.6176) (width 1.6) (layer "F.Cu") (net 4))
 (segment (start 163.668 49.7968) (end 140.1922 49.7968) (width 1.6) (layer "F.Cu") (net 4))
 (segment (start 167.6716 41.656) (end 167.6716 47.8264) (width 1.6) (layer "F.Cu") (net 4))
 (segment (start 167.6716 49.7968) (end 163.668 49.7968) (width 1.6) (layer "F.Cu") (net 4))
 (segment (start 137.192 64.7968) (end 140.1922 64.7968) (width 1.6) (layer "F.Cu") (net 4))
 (segment (start 140.1922 49.7968) (end 137.192 49.7968) (width 1.6) (layer "F.Cu") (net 4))
 (segment (start 140.1922 64.7968) (end 140.1922 49.7968) (width 1.6) (layer "F.Cu") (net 4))
 (segment (start 167.6716 47.8264) (end 189.3448 47.8264) (width 1.6) (layer "F.Cu") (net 4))
 (segment (start 167.6716 47.8264) (end 167.6716 49.7968) (width 1.6) (layer "F.Cu") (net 4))
 (segment (start 189.3448 47.8264) (end 189.3448 54.4984) (width 1.6) (layer "F.Cu") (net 4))
 (segment (start 163.668 55.6176) (end 163.668 49.7968) (width 1.6) (layer "F.Cu") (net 4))
 (segment (start 158.3353 86.8137) (end 158.3353 86.7224) (width 1.6) (layer "F.Cu") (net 3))
 (segment (start 155.7156 86.8137) (end 158.3353 86.8137) (width 1.6) (layer "F.Cu") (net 3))
 (segment (start 189.3448 56.9734) (end 195.4193 56.9734) (width 1.6) (layer "F.Cu") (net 3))
 (via (at 195.4193 56.9734) (size 0.8) (drill 0.4) (layers "F.Cu" "B.Cu") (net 3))
 (via (at 155.7156 86.8137) (size 0.8) (drill 0.4) (layers "F.Cu" "B.Cu") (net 3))
 (segment (start 174.7954 88.6326) (end 174.7954 76.6226) (width 1.6) (layer "B.Cu") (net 3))
 (segment (start 174.7954 76.6226) (end 195.4193 76.6226) (width 1.6) (layer "B.Cu") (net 3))
 (segment (start 155.7156 86.8137) (end 155.7156 88.6326) (width 1.6) (layer "B.Cu") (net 3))
 (segment (start 195.4193 76.6226) (end 195.4193 56.9734) (width 1.6) (layer "B.Cu") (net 3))
 (segment (start 155.7156 88.6326) (end 174.7954 88.6326) (width 1.6) (layer "B.Cu") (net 3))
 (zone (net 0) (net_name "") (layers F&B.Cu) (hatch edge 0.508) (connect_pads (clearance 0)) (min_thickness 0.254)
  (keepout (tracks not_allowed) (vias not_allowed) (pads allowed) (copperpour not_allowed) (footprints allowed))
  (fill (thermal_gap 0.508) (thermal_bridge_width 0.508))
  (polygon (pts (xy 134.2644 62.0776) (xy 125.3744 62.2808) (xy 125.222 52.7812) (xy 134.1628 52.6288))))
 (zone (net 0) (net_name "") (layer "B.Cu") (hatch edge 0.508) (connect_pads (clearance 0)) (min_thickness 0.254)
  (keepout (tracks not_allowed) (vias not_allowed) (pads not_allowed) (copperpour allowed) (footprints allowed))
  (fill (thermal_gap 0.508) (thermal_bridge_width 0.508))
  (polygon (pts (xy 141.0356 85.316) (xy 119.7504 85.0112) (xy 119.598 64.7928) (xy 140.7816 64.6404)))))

